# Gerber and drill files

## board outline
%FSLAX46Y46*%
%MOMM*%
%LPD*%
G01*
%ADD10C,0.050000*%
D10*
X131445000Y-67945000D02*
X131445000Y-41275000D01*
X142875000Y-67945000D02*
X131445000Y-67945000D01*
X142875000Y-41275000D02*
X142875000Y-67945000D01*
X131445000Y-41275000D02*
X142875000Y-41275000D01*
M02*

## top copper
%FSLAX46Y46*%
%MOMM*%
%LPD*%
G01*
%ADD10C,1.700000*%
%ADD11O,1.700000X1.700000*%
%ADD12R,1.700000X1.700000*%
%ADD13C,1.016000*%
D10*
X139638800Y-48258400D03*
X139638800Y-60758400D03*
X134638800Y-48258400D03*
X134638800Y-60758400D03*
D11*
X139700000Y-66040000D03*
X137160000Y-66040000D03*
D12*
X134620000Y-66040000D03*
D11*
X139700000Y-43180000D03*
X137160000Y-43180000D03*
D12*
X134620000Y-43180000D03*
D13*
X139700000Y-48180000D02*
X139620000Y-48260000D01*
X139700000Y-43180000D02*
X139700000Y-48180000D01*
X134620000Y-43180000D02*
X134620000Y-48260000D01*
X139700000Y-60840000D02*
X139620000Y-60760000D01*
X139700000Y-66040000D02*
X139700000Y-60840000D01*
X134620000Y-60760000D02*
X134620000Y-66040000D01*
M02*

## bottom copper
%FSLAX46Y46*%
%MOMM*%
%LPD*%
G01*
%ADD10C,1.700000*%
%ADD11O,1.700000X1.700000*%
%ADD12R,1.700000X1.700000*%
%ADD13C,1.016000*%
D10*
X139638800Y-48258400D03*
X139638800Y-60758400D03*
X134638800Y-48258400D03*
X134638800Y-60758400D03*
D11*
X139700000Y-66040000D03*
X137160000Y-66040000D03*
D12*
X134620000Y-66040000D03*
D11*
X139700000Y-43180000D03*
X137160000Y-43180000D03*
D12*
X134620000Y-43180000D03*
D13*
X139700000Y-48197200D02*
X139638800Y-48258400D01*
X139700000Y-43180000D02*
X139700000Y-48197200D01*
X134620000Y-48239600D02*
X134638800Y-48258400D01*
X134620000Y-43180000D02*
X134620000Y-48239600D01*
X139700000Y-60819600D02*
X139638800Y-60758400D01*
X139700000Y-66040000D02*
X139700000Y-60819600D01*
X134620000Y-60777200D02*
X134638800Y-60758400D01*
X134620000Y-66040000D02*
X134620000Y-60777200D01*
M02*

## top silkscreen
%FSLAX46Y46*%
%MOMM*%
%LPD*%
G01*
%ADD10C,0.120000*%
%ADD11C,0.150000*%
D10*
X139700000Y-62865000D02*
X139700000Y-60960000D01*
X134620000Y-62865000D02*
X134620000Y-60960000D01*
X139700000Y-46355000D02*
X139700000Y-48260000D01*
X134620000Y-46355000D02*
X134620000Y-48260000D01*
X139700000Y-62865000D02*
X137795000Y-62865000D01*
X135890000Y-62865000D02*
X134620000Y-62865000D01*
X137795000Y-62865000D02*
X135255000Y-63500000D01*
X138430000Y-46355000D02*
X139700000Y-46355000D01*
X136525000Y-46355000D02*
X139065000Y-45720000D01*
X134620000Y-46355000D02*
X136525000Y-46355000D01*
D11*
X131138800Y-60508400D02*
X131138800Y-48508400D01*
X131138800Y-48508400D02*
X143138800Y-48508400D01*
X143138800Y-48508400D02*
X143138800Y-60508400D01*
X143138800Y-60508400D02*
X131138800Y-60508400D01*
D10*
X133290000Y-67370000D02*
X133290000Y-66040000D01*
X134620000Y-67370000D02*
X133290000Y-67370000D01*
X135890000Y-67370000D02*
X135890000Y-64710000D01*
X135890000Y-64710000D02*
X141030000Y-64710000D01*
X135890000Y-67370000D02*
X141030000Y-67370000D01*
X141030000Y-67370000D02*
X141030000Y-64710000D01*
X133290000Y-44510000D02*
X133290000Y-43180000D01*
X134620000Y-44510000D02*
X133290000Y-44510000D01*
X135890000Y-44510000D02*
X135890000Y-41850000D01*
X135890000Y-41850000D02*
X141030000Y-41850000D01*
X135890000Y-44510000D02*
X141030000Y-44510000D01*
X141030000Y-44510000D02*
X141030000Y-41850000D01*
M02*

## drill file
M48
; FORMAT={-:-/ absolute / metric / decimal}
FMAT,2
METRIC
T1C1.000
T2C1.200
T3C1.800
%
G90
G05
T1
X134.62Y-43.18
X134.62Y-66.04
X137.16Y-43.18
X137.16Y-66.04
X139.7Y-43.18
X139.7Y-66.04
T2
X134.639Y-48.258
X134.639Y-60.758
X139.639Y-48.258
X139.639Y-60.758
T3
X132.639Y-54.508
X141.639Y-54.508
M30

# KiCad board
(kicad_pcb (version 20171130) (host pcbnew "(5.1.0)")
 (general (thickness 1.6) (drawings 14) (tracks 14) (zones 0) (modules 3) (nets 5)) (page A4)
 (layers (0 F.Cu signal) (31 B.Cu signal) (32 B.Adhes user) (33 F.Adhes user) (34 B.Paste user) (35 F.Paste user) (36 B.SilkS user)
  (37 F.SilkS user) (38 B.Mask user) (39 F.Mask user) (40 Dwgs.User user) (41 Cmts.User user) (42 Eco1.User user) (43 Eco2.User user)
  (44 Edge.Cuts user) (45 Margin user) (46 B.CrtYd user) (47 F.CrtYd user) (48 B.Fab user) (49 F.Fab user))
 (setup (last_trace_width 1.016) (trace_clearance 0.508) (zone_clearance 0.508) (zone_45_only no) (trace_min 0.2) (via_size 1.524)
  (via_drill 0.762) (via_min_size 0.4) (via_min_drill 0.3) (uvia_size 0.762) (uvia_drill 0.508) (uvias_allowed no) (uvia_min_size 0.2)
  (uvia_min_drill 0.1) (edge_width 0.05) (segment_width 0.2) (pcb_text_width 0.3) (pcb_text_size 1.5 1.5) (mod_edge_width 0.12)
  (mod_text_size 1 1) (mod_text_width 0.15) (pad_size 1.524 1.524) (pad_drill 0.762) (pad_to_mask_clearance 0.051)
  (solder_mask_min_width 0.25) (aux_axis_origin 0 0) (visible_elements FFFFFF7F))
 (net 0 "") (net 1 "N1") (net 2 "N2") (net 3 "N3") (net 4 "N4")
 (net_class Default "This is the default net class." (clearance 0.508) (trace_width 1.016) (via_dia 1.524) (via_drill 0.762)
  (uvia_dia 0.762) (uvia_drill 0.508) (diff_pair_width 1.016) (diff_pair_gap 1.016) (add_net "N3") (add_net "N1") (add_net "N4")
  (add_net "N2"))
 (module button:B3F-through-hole (layer F.Cu) (at 137.1388 54.5084 90)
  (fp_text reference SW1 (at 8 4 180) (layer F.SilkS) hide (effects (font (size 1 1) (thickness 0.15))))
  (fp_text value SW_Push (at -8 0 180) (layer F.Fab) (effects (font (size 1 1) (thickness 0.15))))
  (fp_line (start -6 -6) (end 6 -6) (layer F.SilkS) (width 0.15))
  (fp_line (start 6 -6) (end 6 6) (layer F.SilkS) (width 0.15))
  (fp_line (start 6 6) (end -6 6) (layer F.SilkS) (width 0.15))
  (fp_line (start -6 6) (end -6 -6) (layer F.SilkS) (width 0.15))
  (pad 1 thru_hole circle (at 6.25 2.5 90) (size 1.7 1.7) (drill 1.2) (layers *.Cu *.Mask) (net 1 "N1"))
  (pad 2 thru_hole circle (at -6.25 2.5 90) (size 1.7 1.7) (drill 1.2) (layers *.Cu *.Mask) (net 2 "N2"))
  (pad 3 thru_hole circle (at 6.25 -2.5 90) (size 1.7 1.7) (drill 1.2) (layers *.Cu *.Mask) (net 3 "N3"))
  (pad 4 thru_hole circle (at -6.25 -2.5 90) (size 1.7 1.7) (drill 1.2) (layers *.Cu *.Mask) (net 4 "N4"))
  (pad "" np_thru_hole circle (at 0 -4.5 90) (size 1.8 1.8) (drill 1.8) (layers *.Cu *.Mask))
  (pad "" np_thru_hole circle (at 0 4.5 90) (size 1.8 1.8) (drill 1.8) (layers *.Cu *.Mask)))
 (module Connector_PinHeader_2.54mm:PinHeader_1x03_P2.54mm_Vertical (layer F.Cu) (at 134.62 66.04 90)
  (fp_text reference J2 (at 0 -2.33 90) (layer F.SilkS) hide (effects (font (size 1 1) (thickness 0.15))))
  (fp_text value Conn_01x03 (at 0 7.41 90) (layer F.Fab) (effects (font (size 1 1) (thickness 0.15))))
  (fp_line (start -1.33 -1.33) (end 0 -1.33) (layer F.SilkS) (width 0.12))
  (fp_line (start -1.33 0) (end -1.33 -1.33) (layer F.SilkS) (width 0.12))
  (fp_line (start -1.33 1.27) (end 1.33 1.27) (layer F.SilkS) (width 0.12))
  (fp_line (start 1.33 1.27) (end 1.33 6.41) (layer F.SilkS) (width 0.12))
  (fp_line (start -1.33 1.27) (end -1.33 6.41) (layer F.SilkS) (width 0.12))
  (fp_line (start -1.33 6.41) (end 1.33 6.41) (layer F.SilkS) (width 0.12))
  (pad 3 thru_hole oval (at 0 5.08 90) (size 1.7 1.7) (drill 1) (layers *.Cu *.Mask) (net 2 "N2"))
  (pad 2 thru_hole oval (at 0 2.54 90) (size 1.7 1.7) (drill 1) (layers *.Cu *.Mask))
  (pad 1 thru_hole rect (at 0 0 90) (size 1.7 1.7) (drill 1) (layers *.Cu *.Mask) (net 4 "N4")))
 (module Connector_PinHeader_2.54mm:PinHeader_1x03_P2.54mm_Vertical (layer F.Cu) (at 134.62 43.18 90)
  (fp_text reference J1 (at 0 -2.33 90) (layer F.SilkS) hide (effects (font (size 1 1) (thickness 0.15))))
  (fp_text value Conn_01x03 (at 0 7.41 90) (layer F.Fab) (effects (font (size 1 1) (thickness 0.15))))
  (fp_line (start -1.33 -1.33) (end 0 -1.33) (layer F.SilkS) (width 0.12))
  (fp_line (start -1.33 0) (end -1.33 -1.33) (layer F.SilkS) (width 0.12))
  (fp_line (start -1.33 1.27) (end 1.33 1.27) (layer F.SilkS) (width 0.12))
  (fp_line (start 1.33 1.27) (end 1.33 6.41) (layer F.SilkS) (width 0.12))
  (fp_line (start -1.33 1.27) (end -1.33 6.41) (layer F.SilkS) (width 0.12))
  (fp_line (start -1.33 6.41) (end 1.33 6.41) (layer F.SilkS) (width 0.12))
  (pad 3 thru_hole oval (at 0 5.08 90) (size 1.7 1.7) (drill 1) (layers *.Cu *.Mask) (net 1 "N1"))
  (pad 2 thru_hole oval (at 0 2.54 90) (size 1.7 1.7) (drill 1) (layers *.Cu *.Mask))
  (pad 1 thru_hole rect (at 0 0 90) (size 1.7 1.7) (drill 1) (layers *.Cu *.Mask) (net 3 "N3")))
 (gr_line (start 139.7 62.865) (end 139.7 60.96) (layer F.SilkS) (width 0.12))
 (gr_line (start 134.62 62.865) (end 134.62 60.96) (layer F.SilkS) (width 0.12))
 (gr_line (start 139.7 46.355) (end 139.7 48.26) (layer F.SilkS) (width 0.12))
 (gr_line (start 134.62 46.355) (end 134.62 48.26) (layer F.SilkS) (width 0.12))
 (gr_line (start 131.445 67.945) (end 131.445 41.275) (layer Edge.Cuts) (width 0.05))
 (gr_line (start 142.875 67.945) (end 131.445 67.945) (layer Edge.Cuts) (width 0.05))
 (gr_line (start 142.875 41.275) (end 142.875 67.945) (layer Edge.Cuts) (width 0.05))
 (gr_line (start 131.445 41.275) (end 142.875 41.275) (layer Edge.Cuts) (width 0.05))
 (gr_line (start 139.7 62.865) (end 137.795 62.865) (layer F.SilkS) (width 0.12))
 (gr_line (start 135.89 62.865) (end 134.62 62.865) (layer F.SilkS) (width 0.12))
 (gr_line (start 137.795 62.865) (end 135.255 63.5) (layer F.SilkS) (width 0.12))
 (gr_line (start 138.43 46.355) (end 139.7 46.355) (layer F.SilkS) (width 0.12))
 (gr_line (start 136.525 46.355) (end 139.065 45.72) (layer F.SilkS) (width 0.12))
 (gr_line (start 134.62 46.355) (end 136.525 46.355) (layer F.SilkS) (width 0.12))
 (segment (start 139.7 48.18) (end 139.62 48.26) (width 1.016) (layer F.Cu) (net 1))
 (segment (start 139.7 43.18) (end 139.7 48.18) (width 1.016) (layer F.Cu) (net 1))
 (segment (start 139.7 48.1972) (end 139.6388 48.2584) (width 1.016) (layer B.Cu) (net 1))
 (segment (start 139.7 43.18) (end 139.7 48.1972) (width 1.016) (layer B.Cu) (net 1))
 (segment (start 134.62 43.18) (end 134.62 48.26) (width 1.016) (layer F.Cu) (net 3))
 (segment (start 134.62 48.2396) (end 134.6388 48.2584) (width 1.016) (layer B.Cu) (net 3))
 (segment (start 134.62 43.18) (end 134.62 48.2396) (width 1.016) (layer B.Cu) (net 3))
 (segment (start 139.7 60.84) (end 139.62 60.76) (width 1.016) (layer F.Cu) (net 2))
 (segment (start 139.7 66.04) (end 139.7 60.84) (width 1.016) (layer F.Cu) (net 2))
 (segment (start 139.7 60.8196) (end 139.6388 60.7584) (width 1.016) (layer B.Cu) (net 2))
 (segment (start 139.7 66.04) (end 139.7 60.8196) (width 1.016) (layer B.Cu) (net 2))
 (segment (start 134.62 60.76) (end 134.62 66.04) (width 1.016) (layer F.Cu) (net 4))
 (segment (start 134.62 60.7772) (end 134.6388 60.7584) (width 1.016) (layer B.Cu) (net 4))
 (segment (start 134.62 66.04) (end 134.62 60.7772) (width 1.016) (layer B.Cu) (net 4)))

